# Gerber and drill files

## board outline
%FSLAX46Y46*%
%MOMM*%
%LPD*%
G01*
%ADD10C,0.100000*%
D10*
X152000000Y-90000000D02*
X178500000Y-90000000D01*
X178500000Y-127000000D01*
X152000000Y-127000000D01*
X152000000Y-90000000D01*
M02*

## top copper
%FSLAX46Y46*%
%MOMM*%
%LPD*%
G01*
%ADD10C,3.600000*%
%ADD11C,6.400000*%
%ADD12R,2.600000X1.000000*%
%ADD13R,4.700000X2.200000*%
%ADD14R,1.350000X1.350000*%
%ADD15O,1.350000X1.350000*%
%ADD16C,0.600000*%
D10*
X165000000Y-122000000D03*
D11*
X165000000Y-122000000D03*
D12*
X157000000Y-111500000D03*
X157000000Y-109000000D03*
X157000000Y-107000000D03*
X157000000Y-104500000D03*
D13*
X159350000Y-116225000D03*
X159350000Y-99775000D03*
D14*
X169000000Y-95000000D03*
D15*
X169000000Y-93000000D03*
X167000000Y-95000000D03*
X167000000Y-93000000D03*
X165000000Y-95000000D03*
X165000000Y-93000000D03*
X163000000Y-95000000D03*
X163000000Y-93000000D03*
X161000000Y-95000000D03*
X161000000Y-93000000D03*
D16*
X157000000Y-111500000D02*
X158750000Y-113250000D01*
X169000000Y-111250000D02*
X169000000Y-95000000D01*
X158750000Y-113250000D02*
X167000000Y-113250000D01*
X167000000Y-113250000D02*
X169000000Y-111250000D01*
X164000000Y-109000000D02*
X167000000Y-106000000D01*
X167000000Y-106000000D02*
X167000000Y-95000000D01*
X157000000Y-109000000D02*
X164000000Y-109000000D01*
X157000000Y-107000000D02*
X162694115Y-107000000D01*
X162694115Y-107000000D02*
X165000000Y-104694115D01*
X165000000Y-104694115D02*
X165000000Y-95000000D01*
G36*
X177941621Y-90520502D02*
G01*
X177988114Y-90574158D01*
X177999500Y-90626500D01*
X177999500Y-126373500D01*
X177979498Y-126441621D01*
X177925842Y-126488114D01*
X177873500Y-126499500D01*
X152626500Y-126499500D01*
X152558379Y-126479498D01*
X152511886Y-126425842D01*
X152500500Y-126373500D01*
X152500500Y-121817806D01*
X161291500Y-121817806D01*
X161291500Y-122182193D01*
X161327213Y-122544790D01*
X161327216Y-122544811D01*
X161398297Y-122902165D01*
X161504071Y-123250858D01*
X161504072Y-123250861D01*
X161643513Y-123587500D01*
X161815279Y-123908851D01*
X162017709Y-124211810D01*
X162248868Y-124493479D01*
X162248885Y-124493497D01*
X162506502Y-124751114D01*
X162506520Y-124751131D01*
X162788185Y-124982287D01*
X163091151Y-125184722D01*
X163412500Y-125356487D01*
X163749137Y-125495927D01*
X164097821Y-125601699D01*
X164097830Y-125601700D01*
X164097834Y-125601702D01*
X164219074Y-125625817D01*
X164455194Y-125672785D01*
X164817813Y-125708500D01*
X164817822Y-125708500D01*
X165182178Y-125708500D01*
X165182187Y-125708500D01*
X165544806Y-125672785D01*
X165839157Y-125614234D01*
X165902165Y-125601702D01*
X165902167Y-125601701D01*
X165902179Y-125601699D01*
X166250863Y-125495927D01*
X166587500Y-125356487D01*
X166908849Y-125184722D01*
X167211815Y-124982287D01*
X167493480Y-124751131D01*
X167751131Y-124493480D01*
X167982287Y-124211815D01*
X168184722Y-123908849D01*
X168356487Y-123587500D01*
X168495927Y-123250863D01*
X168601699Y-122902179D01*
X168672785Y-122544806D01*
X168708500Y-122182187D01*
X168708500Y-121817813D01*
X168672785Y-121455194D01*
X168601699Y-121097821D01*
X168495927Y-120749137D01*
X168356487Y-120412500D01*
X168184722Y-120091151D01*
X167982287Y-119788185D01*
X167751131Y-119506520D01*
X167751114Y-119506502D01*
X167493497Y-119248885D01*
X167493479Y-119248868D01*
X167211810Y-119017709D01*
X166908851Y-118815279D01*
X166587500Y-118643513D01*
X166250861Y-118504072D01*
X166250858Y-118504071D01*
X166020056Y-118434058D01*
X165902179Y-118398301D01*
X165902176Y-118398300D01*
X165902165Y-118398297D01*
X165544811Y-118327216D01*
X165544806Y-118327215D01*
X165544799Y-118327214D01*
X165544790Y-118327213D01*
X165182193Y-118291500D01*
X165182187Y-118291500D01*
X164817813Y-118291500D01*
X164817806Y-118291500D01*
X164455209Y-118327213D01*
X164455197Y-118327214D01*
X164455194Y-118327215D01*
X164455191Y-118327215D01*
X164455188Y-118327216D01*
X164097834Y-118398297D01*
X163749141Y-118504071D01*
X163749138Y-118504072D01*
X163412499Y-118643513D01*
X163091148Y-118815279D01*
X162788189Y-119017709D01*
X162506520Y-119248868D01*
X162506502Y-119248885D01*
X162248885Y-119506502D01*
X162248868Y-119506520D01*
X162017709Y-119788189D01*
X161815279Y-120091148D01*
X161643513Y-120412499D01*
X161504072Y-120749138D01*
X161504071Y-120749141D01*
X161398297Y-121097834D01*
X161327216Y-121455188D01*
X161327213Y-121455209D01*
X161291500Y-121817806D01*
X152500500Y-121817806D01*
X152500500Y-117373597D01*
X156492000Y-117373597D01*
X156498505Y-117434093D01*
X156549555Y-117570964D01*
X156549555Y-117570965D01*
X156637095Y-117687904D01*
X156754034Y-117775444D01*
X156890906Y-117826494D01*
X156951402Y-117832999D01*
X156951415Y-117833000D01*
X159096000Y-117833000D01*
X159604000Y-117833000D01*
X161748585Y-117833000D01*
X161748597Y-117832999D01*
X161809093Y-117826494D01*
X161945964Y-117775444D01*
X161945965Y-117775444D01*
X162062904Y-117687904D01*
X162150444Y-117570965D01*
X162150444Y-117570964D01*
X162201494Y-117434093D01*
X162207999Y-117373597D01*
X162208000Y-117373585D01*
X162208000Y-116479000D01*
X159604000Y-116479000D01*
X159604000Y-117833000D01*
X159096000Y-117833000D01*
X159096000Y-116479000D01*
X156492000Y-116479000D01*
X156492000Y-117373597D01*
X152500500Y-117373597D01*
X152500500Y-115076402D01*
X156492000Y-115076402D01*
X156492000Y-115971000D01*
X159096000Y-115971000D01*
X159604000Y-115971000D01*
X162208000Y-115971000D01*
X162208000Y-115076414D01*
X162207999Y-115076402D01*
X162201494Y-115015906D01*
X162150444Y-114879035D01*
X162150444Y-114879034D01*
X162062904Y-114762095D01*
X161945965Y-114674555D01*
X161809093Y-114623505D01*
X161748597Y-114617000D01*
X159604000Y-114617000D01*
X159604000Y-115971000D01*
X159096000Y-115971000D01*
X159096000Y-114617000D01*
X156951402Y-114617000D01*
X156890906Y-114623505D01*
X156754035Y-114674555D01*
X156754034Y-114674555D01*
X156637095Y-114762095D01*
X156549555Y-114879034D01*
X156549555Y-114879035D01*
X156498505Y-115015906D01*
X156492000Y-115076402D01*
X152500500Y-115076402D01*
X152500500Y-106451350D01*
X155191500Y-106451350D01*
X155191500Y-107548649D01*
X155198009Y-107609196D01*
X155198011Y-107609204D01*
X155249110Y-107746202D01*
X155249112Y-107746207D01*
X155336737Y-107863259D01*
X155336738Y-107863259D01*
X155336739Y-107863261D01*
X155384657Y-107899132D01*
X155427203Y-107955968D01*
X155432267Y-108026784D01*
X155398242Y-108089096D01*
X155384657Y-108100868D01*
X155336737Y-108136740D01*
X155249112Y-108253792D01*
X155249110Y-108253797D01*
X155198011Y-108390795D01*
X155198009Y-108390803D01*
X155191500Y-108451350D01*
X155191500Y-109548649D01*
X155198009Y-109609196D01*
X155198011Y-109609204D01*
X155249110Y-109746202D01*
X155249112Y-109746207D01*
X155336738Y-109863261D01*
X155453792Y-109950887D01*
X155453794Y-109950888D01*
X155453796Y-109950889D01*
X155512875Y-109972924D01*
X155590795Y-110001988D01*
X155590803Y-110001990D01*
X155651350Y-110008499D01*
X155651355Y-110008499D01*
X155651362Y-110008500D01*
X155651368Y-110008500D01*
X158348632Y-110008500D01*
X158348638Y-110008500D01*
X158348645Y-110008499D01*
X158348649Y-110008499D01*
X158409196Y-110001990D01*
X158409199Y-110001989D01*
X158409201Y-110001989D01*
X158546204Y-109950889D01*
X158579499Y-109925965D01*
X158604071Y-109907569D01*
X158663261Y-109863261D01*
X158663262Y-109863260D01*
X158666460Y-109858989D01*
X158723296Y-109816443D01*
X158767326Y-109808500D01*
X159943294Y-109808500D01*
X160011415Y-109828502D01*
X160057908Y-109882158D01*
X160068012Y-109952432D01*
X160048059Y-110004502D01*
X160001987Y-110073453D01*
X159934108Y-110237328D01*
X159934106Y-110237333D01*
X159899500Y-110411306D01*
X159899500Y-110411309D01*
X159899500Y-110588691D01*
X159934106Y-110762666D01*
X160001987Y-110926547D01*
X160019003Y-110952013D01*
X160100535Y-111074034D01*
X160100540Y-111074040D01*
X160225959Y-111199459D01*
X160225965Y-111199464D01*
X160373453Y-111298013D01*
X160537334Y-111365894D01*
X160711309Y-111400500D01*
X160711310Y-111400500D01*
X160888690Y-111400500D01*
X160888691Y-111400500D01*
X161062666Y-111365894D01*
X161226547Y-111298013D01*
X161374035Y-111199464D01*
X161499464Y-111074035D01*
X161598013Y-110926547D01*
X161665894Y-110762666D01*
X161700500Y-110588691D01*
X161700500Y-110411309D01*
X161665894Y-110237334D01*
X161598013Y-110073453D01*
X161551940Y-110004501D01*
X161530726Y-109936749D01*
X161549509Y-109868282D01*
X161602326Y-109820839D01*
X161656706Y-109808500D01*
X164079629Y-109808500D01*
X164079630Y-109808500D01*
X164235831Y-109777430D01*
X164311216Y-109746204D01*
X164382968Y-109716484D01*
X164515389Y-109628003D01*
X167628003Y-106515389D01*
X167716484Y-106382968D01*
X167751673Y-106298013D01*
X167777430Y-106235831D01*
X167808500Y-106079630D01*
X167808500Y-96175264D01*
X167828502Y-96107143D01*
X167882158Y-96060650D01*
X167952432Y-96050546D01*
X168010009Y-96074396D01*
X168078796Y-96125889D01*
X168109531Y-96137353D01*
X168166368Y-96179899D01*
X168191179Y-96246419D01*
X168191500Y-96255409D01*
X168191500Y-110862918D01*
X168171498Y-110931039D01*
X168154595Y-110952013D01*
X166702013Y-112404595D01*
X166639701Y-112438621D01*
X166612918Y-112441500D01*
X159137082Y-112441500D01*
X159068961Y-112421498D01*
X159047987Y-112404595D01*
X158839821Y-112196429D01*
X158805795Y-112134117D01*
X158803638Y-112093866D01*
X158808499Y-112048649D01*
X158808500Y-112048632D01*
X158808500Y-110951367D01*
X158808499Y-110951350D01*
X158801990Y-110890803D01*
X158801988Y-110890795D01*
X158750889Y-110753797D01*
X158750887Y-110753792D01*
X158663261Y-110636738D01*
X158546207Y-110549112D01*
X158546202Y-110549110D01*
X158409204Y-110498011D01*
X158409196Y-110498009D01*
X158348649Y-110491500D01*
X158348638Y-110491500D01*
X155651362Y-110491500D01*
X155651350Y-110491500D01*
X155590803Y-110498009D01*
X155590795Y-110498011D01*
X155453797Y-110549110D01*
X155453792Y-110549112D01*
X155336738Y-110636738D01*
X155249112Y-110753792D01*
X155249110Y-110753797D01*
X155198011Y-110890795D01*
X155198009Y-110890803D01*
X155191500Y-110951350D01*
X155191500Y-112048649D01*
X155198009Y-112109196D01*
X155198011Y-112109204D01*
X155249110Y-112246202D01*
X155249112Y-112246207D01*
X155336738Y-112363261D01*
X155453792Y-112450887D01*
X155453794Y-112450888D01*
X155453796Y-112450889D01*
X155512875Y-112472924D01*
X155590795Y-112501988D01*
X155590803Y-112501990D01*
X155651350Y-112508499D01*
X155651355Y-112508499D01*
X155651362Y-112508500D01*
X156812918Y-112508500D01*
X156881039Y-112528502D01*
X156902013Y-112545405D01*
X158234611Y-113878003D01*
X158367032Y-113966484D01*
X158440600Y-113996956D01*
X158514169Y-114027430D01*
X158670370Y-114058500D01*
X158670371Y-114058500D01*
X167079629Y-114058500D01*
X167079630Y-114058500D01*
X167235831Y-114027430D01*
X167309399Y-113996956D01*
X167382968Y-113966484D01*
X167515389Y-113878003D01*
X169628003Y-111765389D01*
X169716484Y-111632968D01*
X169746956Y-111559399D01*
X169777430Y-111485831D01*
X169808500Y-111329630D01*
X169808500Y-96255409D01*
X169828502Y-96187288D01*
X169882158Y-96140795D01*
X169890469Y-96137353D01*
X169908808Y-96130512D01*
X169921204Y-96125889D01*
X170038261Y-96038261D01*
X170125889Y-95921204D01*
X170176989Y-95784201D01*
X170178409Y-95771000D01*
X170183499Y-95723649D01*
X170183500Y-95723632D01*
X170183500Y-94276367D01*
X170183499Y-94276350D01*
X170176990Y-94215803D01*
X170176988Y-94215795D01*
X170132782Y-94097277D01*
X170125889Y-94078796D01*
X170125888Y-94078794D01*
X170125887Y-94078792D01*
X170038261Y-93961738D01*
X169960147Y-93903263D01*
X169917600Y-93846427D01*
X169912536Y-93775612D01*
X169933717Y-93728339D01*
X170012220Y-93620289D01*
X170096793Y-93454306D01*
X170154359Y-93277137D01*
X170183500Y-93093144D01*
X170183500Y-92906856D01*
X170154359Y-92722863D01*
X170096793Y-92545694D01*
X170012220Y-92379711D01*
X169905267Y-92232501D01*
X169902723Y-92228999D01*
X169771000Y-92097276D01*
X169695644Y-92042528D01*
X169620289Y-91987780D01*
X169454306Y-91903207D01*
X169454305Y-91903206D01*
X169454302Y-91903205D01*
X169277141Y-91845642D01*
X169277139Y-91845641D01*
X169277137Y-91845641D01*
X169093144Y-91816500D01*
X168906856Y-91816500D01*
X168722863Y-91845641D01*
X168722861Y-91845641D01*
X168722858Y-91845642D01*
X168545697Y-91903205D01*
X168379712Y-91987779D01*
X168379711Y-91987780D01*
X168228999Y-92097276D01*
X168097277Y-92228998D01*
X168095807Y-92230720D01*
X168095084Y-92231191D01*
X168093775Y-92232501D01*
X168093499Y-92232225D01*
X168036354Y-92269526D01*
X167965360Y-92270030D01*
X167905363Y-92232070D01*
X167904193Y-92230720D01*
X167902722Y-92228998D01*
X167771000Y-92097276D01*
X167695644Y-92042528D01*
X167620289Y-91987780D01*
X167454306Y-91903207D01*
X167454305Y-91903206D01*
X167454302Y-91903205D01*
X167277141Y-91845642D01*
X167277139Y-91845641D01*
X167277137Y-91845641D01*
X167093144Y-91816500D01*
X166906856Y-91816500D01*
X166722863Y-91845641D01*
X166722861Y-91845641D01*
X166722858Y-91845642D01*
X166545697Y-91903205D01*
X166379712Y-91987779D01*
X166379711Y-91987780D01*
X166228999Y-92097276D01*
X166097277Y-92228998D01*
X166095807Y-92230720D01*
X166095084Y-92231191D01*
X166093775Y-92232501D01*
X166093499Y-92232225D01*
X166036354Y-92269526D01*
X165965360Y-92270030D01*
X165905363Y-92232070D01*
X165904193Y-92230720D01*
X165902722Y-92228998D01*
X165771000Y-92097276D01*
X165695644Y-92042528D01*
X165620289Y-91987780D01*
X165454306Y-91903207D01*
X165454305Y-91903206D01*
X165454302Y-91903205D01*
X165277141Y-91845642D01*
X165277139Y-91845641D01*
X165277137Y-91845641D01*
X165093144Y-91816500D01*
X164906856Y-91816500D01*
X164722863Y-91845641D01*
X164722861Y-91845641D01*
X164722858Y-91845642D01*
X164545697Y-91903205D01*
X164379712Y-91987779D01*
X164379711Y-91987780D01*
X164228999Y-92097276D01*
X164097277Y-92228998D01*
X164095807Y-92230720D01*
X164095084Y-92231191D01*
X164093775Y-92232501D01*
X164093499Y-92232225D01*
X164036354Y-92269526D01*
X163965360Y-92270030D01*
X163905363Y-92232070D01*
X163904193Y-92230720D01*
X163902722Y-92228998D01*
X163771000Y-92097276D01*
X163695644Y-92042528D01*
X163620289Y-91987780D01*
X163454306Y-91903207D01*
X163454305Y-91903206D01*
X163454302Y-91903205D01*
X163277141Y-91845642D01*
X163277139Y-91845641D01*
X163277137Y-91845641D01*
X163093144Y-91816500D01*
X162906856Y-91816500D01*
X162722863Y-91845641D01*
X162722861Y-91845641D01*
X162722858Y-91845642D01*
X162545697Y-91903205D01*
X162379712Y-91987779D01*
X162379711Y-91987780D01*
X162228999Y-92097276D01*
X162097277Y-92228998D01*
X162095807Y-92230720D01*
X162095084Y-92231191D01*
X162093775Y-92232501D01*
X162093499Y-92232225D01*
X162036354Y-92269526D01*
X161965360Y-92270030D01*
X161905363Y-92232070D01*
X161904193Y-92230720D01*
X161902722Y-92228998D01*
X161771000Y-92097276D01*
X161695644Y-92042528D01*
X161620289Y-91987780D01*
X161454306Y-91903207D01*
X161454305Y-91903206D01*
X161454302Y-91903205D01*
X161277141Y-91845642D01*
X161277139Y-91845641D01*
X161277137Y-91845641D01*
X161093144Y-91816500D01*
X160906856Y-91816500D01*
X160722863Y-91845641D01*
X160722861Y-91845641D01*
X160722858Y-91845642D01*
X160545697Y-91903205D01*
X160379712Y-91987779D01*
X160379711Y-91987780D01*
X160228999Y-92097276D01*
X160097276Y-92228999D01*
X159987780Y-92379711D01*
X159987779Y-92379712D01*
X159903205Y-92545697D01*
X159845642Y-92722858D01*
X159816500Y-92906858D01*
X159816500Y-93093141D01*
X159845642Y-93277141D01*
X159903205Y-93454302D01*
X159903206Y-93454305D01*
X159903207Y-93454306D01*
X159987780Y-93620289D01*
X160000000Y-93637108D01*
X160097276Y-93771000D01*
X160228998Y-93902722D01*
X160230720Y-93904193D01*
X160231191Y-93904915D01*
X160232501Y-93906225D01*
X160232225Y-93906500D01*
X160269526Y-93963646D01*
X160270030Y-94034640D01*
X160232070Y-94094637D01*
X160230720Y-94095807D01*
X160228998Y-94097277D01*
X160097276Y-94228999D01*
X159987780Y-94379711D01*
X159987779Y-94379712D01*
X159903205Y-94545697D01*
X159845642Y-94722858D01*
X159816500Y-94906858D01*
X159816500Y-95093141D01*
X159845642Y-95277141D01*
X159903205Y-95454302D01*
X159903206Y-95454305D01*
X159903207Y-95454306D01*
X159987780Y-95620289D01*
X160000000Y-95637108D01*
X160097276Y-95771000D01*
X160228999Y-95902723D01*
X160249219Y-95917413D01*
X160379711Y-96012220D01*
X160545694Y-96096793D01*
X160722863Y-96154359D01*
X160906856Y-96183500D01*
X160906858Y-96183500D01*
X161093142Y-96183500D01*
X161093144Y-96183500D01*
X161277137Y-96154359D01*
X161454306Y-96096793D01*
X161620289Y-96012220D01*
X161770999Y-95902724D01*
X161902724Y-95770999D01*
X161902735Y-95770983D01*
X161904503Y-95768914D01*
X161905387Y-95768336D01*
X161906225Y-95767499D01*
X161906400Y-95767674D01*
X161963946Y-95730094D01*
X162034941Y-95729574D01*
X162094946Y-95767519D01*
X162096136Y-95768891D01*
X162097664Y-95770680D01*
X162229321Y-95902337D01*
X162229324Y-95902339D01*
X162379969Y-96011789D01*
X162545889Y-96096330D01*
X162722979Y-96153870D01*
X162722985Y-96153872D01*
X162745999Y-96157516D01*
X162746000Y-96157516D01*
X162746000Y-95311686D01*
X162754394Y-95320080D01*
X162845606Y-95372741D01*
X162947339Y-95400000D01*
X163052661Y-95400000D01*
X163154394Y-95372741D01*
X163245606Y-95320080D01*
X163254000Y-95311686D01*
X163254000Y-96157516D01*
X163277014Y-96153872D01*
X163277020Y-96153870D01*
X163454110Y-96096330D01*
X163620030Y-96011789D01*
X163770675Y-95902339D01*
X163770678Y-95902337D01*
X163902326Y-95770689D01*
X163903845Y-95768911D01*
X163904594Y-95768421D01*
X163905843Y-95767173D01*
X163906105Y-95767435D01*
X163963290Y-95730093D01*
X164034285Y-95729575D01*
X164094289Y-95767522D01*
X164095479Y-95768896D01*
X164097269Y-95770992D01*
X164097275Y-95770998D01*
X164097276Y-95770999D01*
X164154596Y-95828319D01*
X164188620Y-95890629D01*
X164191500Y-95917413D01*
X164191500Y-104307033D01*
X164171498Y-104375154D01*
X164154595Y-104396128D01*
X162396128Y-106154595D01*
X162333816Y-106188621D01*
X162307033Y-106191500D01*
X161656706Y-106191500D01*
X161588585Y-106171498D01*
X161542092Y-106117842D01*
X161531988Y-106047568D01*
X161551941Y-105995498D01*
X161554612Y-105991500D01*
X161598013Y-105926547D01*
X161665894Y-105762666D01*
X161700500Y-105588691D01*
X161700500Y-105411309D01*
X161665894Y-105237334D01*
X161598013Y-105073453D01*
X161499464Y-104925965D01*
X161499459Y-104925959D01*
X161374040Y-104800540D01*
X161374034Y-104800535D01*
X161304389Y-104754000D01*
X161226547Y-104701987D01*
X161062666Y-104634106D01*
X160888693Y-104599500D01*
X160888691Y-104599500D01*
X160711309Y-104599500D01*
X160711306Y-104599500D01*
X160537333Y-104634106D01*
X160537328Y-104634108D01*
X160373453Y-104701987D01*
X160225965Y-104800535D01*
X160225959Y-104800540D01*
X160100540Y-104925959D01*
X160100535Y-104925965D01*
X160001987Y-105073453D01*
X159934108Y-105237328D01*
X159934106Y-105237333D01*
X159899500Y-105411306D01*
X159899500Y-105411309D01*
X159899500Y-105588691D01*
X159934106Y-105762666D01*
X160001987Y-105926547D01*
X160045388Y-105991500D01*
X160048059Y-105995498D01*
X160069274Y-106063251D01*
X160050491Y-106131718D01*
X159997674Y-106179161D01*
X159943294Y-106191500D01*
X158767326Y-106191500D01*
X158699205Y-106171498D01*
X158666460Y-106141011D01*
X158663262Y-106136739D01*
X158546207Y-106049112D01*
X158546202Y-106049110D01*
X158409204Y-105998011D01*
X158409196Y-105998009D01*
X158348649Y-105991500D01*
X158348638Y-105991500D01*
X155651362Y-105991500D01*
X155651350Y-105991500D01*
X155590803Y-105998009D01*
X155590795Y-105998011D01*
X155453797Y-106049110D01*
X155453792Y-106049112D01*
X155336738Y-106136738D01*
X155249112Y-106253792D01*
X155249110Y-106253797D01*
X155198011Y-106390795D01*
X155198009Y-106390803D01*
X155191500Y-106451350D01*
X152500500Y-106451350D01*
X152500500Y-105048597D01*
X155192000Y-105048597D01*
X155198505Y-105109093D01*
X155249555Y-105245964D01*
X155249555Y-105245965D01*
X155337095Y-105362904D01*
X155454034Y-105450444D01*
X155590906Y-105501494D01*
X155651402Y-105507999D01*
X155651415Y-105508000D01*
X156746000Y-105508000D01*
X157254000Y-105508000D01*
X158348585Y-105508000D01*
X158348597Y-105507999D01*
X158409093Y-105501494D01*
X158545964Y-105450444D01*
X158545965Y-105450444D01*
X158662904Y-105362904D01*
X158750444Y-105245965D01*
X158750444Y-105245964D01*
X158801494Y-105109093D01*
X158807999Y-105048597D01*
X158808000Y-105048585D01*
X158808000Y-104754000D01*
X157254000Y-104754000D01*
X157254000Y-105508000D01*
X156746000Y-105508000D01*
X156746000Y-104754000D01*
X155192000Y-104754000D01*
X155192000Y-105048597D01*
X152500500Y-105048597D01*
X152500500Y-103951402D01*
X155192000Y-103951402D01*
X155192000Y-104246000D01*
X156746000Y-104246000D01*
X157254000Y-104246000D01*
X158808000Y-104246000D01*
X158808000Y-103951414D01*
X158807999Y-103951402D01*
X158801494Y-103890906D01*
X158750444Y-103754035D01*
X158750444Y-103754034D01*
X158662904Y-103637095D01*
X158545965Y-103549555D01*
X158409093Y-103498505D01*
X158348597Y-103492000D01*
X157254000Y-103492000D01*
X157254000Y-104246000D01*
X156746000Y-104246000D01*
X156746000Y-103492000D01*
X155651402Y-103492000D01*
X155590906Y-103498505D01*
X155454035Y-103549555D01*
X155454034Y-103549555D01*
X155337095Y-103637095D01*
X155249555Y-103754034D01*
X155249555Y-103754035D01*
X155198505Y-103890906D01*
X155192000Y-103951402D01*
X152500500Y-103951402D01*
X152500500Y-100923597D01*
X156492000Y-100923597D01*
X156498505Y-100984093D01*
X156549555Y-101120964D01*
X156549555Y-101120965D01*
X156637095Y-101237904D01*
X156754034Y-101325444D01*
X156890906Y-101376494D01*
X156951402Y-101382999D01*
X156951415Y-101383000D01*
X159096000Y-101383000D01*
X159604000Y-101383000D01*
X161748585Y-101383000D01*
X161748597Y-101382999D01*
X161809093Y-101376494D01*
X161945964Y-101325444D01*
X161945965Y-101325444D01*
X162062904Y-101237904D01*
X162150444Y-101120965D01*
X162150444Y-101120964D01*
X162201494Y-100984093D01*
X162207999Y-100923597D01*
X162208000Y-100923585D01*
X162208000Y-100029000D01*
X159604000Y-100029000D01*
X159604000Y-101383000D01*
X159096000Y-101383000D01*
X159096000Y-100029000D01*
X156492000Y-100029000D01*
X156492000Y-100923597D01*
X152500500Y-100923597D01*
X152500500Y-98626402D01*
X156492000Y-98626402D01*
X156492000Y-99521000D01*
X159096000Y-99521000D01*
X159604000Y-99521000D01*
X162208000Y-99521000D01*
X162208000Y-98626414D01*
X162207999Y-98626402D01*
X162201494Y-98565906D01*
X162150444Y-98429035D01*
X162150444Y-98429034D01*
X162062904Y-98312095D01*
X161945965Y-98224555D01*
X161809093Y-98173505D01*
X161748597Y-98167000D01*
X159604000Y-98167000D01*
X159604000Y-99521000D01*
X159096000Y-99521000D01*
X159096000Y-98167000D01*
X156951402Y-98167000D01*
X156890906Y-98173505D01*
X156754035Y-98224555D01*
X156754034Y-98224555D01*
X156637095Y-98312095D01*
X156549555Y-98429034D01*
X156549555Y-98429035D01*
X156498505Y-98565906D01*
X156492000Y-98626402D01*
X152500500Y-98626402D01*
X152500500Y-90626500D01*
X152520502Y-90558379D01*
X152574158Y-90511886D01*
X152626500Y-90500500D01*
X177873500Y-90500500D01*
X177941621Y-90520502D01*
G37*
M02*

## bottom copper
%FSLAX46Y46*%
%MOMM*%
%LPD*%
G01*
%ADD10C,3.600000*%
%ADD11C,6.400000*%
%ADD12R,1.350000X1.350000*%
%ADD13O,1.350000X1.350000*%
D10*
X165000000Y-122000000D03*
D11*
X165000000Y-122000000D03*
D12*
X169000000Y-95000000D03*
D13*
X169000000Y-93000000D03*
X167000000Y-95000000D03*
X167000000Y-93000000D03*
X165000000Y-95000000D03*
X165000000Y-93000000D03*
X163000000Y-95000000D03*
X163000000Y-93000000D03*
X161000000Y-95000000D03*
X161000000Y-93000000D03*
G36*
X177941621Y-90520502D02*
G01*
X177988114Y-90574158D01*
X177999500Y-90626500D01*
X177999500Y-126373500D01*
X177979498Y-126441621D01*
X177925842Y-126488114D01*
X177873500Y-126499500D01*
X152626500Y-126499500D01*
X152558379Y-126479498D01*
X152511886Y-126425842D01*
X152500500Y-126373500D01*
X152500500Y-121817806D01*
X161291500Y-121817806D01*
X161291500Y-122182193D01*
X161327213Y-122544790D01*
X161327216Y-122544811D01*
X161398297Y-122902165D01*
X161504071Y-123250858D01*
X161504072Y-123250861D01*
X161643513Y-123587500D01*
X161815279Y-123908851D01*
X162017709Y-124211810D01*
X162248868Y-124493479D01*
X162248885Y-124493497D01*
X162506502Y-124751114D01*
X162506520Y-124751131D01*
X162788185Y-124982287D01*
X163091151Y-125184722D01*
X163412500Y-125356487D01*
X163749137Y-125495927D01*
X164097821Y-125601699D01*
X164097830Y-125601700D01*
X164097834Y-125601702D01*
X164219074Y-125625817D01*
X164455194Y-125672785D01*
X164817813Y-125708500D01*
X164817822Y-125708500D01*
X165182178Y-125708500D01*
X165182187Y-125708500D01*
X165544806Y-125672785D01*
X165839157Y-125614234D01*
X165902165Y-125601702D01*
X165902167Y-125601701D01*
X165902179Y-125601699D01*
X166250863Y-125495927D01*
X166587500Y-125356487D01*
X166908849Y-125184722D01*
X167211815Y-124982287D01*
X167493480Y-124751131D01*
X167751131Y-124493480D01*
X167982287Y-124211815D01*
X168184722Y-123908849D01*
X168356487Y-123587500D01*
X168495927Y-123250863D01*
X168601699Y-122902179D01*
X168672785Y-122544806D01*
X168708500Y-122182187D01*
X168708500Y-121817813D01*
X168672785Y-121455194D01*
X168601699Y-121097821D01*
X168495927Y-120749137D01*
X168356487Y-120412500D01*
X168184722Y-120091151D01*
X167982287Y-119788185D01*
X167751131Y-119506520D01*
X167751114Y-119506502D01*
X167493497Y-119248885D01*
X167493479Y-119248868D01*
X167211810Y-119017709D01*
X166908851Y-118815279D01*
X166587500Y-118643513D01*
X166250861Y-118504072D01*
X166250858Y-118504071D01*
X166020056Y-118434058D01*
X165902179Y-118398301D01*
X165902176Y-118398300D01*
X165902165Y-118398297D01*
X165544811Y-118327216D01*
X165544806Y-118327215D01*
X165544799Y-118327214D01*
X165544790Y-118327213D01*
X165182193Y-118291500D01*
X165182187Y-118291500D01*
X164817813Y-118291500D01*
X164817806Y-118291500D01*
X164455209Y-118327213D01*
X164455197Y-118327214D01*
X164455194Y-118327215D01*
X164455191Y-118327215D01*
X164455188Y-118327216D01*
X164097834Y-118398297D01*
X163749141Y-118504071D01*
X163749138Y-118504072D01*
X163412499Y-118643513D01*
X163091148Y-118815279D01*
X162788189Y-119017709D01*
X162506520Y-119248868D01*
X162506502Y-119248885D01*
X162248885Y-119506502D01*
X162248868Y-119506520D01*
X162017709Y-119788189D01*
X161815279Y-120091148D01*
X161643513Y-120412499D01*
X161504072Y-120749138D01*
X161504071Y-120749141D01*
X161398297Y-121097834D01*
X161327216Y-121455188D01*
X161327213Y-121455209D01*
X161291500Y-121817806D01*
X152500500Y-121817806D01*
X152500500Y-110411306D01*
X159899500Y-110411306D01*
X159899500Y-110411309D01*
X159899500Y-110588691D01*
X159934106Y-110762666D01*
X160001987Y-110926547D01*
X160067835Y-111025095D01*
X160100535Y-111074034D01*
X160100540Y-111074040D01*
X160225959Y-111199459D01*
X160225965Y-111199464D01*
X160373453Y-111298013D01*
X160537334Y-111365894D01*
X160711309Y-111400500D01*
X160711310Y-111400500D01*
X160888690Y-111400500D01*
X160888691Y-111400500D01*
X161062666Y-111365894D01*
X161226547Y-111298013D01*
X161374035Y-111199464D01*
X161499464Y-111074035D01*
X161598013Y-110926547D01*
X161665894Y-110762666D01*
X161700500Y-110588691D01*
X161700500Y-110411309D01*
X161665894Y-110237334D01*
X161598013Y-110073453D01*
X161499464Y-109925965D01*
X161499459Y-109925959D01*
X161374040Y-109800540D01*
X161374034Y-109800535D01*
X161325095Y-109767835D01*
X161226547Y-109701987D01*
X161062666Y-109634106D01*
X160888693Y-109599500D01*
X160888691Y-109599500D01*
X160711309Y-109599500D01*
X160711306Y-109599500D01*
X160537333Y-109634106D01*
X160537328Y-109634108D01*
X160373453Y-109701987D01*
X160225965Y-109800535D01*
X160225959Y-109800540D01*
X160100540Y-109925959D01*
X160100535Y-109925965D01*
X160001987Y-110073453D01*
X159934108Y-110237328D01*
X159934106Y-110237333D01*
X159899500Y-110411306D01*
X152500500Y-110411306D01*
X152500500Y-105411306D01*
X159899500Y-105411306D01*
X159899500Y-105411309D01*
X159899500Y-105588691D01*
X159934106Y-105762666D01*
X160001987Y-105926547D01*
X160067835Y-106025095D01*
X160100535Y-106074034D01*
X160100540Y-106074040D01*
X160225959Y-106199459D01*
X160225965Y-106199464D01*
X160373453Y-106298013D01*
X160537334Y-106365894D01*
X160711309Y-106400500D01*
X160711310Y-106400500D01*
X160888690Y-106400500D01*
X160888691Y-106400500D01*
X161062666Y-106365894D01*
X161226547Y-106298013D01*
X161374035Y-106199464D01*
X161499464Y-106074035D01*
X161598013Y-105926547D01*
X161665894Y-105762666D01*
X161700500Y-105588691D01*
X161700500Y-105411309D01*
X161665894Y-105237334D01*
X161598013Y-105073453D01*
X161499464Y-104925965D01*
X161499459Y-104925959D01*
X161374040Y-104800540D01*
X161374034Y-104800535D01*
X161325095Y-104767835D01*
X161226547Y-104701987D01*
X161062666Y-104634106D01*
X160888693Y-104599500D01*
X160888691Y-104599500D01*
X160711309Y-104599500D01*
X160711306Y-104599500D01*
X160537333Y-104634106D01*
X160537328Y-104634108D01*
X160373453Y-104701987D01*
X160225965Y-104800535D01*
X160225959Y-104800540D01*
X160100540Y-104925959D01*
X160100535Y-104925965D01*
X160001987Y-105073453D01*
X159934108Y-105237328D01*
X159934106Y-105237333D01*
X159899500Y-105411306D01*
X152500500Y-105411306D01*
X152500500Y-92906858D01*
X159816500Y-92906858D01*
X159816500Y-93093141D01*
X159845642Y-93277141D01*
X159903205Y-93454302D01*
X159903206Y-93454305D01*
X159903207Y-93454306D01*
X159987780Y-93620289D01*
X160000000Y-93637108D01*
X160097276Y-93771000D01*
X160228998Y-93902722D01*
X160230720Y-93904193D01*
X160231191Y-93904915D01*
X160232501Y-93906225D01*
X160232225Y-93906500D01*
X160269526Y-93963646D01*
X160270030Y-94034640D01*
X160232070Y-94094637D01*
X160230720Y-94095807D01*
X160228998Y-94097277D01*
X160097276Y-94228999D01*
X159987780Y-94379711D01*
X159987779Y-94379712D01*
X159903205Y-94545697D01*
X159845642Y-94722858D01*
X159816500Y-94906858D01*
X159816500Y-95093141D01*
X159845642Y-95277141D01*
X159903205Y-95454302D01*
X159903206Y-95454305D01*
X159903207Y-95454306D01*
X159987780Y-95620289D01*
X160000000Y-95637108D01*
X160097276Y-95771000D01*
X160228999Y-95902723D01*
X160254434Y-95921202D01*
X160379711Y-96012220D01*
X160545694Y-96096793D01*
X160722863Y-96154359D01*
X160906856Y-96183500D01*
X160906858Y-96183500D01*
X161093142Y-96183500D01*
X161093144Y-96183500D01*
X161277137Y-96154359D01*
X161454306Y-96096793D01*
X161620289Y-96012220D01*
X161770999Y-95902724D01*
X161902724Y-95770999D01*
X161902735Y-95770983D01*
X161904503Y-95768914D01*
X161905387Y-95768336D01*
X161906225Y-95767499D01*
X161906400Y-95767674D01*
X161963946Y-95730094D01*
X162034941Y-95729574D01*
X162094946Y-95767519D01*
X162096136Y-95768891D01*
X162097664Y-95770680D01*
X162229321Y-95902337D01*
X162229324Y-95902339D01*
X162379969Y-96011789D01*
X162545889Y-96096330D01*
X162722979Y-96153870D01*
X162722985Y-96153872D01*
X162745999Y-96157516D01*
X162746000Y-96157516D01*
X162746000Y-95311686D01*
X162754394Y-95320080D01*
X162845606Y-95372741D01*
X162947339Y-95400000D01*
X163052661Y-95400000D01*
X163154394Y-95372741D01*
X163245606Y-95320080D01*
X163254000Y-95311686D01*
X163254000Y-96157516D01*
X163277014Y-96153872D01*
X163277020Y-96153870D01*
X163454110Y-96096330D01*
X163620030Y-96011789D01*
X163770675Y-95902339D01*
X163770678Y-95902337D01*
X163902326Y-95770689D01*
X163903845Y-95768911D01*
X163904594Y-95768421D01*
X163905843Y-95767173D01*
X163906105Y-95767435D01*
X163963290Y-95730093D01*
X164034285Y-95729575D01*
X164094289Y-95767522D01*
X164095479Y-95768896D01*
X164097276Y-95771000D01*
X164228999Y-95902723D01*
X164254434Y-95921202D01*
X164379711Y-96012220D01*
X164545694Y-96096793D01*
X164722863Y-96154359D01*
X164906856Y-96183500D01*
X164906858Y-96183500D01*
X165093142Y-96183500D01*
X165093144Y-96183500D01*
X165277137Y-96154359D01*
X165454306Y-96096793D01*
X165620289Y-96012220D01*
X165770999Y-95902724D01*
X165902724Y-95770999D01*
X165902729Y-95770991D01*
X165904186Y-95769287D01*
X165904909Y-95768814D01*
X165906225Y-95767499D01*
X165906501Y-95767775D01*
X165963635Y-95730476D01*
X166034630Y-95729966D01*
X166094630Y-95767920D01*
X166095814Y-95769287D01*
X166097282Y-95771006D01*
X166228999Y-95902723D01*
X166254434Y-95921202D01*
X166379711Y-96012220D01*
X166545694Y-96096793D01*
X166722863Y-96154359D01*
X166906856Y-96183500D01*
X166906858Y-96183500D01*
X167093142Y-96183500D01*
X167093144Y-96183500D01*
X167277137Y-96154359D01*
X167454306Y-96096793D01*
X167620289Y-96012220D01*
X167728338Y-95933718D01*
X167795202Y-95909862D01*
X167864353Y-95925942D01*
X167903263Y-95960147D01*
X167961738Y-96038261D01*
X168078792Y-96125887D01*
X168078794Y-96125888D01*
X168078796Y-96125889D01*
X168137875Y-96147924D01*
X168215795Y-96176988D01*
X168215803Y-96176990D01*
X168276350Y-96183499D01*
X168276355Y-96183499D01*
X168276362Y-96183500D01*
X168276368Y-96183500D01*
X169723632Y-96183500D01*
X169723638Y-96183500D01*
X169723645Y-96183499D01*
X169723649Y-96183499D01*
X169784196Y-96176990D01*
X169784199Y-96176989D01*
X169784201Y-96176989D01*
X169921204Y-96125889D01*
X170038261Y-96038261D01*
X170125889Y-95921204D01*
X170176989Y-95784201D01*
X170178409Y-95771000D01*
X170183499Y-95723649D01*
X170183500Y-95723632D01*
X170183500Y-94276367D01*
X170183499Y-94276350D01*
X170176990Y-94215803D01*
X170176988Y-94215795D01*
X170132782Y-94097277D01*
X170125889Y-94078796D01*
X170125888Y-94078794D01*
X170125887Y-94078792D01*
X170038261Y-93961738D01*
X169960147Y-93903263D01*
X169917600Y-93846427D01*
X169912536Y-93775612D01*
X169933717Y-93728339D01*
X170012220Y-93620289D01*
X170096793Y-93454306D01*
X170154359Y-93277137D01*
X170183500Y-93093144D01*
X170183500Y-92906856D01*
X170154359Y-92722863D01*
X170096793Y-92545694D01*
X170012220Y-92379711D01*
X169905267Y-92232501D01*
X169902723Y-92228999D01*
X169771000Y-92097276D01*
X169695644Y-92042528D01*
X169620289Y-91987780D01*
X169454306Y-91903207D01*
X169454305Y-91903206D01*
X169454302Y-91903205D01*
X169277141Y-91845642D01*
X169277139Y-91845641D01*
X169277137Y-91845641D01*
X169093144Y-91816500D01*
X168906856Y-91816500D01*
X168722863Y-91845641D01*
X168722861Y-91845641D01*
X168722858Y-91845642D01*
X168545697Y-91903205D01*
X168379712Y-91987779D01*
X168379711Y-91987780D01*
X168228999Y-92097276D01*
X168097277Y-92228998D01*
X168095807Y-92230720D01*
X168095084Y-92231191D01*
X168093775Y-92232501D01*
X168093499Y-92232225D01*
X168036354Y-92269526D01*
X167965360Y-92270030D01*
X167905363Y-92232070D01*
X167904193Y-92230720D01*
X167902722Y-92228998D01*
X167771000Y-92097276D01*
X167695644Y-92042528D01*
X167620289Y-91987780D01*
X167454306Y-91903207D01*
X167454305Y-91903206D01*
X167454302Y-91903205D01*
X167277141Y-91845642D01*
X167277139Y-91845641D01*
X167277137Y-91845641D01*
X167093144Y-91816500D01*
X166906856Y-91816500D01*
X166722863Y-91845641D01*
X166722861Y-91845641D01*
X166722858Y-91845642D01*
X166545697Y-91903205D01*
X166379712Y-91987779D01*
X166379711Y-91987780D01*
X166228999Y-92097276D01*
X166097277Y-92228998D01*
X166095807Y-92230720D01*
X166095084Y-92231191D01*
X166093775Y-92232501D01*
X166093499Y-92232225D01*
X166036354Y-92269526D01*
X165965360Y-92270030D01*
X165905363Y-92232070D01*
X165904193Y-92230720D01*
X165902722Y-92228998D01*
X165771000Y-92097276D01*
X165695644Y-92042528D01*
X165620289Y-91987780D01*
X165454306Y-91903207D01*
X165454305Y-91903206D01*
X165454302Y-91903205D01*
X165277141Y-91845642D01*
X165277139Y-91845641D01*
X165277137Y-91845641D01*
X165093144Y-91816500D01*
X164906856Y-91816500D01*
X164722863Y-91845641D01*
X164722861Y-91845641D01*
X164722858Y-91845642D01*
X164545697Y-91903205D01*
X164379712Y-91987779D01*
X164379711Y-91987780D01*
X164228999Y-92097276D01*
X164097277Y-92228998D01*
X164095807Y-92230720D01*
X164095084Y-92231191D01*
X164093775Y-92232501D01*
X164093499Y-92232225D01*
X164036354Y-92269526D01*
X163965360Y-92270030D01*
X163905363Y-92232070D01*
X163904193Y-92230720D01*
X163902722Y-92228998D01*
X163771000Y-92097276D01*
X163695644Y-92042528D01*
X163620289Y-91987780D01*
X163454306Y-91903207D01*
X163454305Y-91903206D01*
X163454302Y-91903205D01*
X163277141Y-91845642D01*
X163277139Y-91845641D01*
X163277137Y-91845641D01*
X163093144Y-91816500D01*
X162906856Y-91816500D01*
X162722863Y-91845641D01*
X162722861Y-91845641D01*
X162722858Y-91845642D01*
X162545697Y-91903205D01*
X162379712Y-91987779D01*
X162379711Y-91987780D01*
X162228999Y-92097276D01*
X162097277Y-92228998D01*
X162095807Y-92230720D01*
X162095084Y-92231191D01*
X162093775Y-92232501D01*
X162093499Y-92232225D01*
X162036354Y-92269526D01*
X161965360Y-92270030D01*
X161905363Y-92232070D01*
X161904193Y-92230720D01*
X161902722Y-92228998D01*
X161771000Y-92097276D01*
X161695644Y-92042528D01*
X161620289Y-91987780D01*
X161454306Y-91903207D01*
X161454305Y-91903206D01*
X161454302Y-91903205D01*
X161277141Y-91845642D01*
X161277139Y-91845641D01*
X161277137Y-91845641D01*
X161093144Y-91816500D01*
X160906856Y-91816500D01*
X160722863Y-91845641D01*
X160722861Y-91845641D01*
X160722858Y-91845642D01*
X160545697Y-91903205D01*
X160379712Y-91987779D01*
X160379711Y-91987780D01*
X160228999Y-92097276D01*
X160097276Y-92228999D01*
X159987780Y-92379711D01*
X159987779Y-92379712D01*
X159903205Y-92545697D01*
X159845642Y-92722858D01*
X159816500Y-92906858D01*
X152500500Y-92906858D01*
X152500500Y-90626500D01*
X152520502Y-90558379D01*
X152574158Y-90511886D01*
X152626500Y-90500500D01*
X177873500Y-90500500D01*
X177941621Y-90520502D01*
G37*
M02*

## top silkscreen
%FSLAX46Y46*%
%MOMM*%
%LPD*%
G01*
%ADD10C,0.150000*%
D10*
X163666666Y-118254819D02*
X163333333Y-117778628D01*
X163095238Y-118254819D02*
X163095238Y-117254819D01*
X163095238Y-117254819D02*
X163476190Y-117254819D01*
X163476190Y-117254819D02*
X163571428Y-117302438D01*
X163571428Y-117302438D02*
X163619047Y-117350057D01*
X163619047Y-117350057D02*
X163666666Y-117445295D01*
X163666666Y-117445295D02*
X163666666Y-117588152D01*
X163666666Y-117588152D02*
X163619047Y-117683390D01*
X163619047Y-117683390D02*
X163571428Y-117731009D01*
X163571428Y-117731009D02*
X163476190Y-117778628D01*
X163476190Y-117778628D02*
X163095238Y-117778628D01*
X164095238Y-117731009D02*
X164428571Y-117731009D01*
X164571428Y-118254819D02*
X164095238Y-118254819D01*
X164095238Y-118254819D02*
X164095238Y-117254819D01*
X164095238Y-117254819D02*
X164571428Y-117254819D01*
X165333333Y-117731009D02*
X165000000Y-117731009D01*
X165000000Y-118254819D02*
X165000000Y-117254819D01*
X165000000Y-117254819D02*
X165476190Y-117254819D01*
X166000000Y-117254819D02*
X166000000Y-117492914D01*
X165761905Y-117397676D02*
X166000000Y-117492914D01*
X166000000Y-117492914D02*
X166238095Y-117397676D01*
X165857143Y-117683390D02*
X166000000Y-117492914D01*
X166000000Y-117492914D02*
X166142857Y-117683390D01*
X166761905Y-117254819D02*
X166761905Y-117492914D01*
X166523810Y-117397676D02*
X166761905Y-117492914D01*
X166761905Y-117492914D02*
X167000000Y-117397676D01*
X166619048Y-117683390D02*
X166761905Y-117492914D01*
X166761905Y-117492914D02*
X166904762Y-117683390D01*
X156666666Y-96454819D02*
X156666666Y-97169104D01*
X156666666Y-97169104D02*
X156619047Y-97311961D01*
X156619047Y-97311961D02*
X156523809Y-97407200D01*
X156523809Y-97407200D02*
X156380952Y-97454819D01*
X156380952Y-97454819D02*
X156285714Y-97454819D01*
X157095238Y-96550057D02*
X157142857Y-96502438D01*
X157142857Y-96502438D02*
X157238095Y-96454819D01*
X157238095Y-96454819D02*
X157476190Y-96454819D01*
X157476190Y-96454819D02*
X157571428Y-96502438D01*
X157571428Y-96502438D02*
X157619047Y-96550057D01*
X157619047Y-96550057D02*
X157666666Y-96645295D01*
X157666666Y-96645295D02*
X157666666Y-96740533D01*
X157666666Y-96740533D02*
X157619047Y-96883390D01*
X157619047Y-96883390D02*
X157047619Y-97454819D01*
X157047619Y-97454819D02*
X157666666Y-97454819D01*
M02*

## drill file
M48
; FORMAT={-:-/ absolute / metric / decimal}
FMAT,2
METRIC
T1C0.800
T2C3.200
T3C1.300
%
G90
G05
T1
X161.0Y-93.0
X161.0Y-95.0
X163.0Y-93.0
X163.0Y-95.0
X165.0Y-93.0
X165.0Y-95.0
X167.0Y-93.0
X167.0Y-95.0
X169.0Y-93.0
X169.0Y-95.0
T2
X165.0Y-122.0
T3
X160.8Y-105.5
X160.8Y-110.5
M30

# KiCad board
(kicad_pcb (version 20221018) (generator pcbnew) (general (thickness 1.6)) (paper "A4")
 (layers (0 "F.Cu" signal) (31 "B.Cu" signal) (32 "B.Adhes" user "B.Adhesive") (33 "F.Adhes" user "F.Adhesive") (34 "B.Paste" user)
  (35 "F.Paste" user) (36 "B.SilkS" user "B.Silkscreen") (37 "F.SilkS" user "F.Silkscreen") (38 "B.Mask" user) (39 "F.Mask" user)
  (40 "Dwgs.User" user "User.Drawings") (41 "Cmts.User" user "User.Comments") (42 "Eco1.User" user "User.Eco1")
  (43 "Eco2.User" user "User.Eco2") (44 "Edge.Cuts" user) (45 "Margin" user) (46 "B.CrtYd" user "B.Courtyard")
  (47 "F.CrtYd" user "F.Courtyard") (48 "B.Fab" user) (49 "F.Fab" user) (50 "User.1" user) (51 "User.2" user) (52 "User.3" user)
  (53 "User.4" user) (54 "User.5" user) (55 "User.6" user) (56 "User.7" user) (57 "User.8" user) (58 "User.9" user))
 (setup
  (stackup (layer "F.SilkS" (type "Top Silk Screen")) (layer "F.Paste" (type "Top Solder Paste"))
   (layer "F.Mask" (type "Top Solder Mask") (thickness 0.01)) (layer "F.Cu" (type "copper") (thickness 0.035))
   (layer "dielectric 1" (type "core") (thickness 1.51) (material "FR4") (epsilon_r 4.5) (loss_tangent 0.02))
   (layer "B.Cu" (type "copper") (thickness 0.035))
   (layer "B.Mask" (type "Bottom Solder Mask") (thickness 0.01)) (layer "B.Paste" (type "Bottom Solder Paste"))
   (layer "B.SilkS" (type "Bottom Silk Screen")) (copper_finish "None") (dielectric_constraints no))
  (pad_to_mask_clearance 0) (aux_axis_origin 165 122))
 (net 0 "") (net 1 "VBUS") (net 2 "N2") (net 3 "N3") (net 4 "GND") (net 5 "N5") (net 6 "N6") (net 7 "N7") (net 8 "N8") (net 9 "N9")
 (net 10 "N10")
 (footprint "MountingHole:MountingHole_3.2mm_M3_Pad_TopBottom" (layer "F.Cu") (at 165 122)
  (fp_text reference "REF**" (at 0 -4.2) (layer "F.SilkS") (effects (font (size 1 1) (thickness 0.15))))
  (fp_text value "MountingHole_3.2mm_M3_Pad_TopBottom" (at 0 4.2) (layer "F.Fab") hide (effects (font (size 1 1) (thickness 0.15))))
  (pad "1" thru_hole circle (at 0 0) (size 3.6 3.6) (drill 3.2) (layers *.Cu *.Mask))
  (pad "1" connect circle (at 0 0) (size 6.4 6.4) (layers "F.Cu" "F.Mask"))
  (pad "1" connect circle (at 0 0) (size 6.4 6.4) (layers "B.Cu" "B.Mask")))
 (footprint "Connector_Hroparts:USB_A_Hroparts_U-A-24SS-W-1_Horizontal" (layer "F.Cu") (at 159.35 108 90)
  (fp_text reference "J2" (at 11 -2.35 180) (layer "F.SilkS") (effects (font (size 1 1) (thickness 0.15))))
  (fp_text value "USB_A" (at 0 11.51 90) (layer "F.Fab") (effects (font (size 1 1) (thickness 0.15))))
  (pad "" np_thru_hole circle (at -2.5 1.45 90) (size 1 1) (drill 1.3) (layers F&B.Cu *.Mask))
  (pad "" np_thru_hole circle (at 2.5 1.45 90) (size 1 1) (drill 1.3) (layers F&B.Cu *.Mask))
  (pad "1" smd rect (at -3.5 -2.35 90) (size 1 2.6) (layers "F.Cu" "F.Paste" "F.Mask") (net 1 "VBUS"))
  (pad "2" smd rect (at -1 -2.35 90) (size 1 2.6) (layers "F.Cu" "F.Paste" "F.Mask") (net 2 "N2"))
  (pad "3" smd rect (at 1 -2.35 90) (size 1 2.6) (layers "F.Cu" "F.Paste" "F.Mask") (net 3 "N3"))
  (pad "4" smd rect (at 3.5 -2.35 90) (size 1 2.6) (layers "F.Cu" "F.Paste" "F.Mask") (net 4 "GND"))
  (pad "5" smd rect (at -8.225 0 90) (size 2.2 4.7) (layers "F.Cu" "F.Paste" "F.Mask") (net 4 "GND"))
  (pad "5" smd rect (at 8.225 0 90) (size 2.2 4.7) (layers "F.Cu" "F.Paste" "F.Mask") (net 4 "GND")))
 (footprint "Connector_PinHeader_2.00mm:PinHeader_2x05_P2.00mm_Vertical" (layer "B.Cu") (at 169 95 90)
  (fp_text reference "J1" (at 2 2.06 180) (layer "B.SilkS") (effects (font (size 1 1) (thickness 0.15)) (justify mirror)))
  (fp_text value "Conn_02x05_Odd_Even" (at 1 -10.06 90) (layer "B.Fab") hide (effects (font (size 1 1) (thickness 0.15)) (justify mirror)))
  (pad "1" thru_hole rect (at 0 0 90) (size 1.35 1.35) (drill 0.8) (layers *.Cu *.Mask) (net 1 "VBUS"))
  (pad "2" thru_hole oval (at 2 0 90) (size 1.35 1.35) (drill 0.8) (layers *.Cu *.Mask) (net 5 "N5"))
  (pad "3" thru_hole oval (at 0 -2 90) (size 1.35 1.35) (drill 0.8) (layers *.Cu *.Mask) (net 2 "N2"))
  (pad "4" thru_hole oval (at 2 -2 90) (size 1.35 1.35) (drill 0.8) (layers *.Cu *.Mask) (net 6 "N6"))
  (pad "5" thru_hole oval (at 0 -4 90) (size 1.35 1.35) (drill 0.8) (layers *.Cu *.Mask) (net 3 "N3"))
  (pad "6" thru_hole oval (at 2 -4 90) (size 1.35 1.35) (drill 0.8) (layers *.Cu *.Mask) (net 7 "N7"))
  (pad "7" thru_hole oval (at 0 -6 90) (size 1.35 1.35) (drill 0.8) (layers *.Cu *.Mask) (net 4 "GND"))
  (pad "8" thru_hole oval (at 2 -6 90) (size 1.35 1.35) (drill 0.8) (layers *.Cu *.Mask) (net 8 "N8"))
  (pad "9" thru_hole oval (at 0 -8 90) (size 1.35 1.35) (drill 0.8) (layers *.Cu *.Mask) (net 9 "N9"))
  (pad "10" thru_hole oval (at 2 -8 90) (size 1.35 1.35) (drill 0.8) (layers *.Cu *.Mask) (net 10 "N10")))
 (gr_rect (start 152 90) (end 178.5 127) (stroke (width 0.1) (type default)) (fill none) (layer "Edge.Cuts"))
 (segment (start 157 111.5) (end 158.75 113.25) (width 0.6) (layer "F.Cu") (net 1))
 (segment (start 169 111.25) (end 169 95) (width 0.6) (layer "F.Cu") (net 1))
 (segment (start 158.75 113.25) (end 167 113.25) (width 0.6) (layer "F.Cu") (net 1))
 (segment (start 167 113.25) (end 169 111.25) (width 0.6) (layer "F.Cu") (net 1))
 (segment (start 164 109) (end 167 106) (width 0.6) (layer "F.Cu") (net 2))
 (segment (start 167 106) (end 167 95) (width 0.6) (layer "F.Cu") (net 2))
 (segment (start 157 109) (end 164 109) (width 0.6) (layer "F.Cu") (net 2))
 (segment (start 157 107) (end 162.694115 107) (width 0.6) (layer "F.Cu") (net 3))
 (segment (start 162.694115 107) (end 165 104.694115) (width 0.6) (layer "F.Cu") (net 3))
 (segment (start 165 104.694115) (end 165 95) (width 0.6) (layer "F.Cu") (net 3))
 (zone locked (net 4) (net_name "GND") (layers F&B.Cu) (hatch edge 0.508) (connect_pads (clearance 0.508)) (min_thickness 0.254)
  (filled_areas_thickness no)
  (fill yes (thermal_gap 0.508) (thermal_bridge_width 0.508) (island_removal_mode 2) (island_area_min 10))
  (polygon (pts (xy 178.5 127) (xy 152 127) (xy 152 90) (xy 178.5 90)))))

